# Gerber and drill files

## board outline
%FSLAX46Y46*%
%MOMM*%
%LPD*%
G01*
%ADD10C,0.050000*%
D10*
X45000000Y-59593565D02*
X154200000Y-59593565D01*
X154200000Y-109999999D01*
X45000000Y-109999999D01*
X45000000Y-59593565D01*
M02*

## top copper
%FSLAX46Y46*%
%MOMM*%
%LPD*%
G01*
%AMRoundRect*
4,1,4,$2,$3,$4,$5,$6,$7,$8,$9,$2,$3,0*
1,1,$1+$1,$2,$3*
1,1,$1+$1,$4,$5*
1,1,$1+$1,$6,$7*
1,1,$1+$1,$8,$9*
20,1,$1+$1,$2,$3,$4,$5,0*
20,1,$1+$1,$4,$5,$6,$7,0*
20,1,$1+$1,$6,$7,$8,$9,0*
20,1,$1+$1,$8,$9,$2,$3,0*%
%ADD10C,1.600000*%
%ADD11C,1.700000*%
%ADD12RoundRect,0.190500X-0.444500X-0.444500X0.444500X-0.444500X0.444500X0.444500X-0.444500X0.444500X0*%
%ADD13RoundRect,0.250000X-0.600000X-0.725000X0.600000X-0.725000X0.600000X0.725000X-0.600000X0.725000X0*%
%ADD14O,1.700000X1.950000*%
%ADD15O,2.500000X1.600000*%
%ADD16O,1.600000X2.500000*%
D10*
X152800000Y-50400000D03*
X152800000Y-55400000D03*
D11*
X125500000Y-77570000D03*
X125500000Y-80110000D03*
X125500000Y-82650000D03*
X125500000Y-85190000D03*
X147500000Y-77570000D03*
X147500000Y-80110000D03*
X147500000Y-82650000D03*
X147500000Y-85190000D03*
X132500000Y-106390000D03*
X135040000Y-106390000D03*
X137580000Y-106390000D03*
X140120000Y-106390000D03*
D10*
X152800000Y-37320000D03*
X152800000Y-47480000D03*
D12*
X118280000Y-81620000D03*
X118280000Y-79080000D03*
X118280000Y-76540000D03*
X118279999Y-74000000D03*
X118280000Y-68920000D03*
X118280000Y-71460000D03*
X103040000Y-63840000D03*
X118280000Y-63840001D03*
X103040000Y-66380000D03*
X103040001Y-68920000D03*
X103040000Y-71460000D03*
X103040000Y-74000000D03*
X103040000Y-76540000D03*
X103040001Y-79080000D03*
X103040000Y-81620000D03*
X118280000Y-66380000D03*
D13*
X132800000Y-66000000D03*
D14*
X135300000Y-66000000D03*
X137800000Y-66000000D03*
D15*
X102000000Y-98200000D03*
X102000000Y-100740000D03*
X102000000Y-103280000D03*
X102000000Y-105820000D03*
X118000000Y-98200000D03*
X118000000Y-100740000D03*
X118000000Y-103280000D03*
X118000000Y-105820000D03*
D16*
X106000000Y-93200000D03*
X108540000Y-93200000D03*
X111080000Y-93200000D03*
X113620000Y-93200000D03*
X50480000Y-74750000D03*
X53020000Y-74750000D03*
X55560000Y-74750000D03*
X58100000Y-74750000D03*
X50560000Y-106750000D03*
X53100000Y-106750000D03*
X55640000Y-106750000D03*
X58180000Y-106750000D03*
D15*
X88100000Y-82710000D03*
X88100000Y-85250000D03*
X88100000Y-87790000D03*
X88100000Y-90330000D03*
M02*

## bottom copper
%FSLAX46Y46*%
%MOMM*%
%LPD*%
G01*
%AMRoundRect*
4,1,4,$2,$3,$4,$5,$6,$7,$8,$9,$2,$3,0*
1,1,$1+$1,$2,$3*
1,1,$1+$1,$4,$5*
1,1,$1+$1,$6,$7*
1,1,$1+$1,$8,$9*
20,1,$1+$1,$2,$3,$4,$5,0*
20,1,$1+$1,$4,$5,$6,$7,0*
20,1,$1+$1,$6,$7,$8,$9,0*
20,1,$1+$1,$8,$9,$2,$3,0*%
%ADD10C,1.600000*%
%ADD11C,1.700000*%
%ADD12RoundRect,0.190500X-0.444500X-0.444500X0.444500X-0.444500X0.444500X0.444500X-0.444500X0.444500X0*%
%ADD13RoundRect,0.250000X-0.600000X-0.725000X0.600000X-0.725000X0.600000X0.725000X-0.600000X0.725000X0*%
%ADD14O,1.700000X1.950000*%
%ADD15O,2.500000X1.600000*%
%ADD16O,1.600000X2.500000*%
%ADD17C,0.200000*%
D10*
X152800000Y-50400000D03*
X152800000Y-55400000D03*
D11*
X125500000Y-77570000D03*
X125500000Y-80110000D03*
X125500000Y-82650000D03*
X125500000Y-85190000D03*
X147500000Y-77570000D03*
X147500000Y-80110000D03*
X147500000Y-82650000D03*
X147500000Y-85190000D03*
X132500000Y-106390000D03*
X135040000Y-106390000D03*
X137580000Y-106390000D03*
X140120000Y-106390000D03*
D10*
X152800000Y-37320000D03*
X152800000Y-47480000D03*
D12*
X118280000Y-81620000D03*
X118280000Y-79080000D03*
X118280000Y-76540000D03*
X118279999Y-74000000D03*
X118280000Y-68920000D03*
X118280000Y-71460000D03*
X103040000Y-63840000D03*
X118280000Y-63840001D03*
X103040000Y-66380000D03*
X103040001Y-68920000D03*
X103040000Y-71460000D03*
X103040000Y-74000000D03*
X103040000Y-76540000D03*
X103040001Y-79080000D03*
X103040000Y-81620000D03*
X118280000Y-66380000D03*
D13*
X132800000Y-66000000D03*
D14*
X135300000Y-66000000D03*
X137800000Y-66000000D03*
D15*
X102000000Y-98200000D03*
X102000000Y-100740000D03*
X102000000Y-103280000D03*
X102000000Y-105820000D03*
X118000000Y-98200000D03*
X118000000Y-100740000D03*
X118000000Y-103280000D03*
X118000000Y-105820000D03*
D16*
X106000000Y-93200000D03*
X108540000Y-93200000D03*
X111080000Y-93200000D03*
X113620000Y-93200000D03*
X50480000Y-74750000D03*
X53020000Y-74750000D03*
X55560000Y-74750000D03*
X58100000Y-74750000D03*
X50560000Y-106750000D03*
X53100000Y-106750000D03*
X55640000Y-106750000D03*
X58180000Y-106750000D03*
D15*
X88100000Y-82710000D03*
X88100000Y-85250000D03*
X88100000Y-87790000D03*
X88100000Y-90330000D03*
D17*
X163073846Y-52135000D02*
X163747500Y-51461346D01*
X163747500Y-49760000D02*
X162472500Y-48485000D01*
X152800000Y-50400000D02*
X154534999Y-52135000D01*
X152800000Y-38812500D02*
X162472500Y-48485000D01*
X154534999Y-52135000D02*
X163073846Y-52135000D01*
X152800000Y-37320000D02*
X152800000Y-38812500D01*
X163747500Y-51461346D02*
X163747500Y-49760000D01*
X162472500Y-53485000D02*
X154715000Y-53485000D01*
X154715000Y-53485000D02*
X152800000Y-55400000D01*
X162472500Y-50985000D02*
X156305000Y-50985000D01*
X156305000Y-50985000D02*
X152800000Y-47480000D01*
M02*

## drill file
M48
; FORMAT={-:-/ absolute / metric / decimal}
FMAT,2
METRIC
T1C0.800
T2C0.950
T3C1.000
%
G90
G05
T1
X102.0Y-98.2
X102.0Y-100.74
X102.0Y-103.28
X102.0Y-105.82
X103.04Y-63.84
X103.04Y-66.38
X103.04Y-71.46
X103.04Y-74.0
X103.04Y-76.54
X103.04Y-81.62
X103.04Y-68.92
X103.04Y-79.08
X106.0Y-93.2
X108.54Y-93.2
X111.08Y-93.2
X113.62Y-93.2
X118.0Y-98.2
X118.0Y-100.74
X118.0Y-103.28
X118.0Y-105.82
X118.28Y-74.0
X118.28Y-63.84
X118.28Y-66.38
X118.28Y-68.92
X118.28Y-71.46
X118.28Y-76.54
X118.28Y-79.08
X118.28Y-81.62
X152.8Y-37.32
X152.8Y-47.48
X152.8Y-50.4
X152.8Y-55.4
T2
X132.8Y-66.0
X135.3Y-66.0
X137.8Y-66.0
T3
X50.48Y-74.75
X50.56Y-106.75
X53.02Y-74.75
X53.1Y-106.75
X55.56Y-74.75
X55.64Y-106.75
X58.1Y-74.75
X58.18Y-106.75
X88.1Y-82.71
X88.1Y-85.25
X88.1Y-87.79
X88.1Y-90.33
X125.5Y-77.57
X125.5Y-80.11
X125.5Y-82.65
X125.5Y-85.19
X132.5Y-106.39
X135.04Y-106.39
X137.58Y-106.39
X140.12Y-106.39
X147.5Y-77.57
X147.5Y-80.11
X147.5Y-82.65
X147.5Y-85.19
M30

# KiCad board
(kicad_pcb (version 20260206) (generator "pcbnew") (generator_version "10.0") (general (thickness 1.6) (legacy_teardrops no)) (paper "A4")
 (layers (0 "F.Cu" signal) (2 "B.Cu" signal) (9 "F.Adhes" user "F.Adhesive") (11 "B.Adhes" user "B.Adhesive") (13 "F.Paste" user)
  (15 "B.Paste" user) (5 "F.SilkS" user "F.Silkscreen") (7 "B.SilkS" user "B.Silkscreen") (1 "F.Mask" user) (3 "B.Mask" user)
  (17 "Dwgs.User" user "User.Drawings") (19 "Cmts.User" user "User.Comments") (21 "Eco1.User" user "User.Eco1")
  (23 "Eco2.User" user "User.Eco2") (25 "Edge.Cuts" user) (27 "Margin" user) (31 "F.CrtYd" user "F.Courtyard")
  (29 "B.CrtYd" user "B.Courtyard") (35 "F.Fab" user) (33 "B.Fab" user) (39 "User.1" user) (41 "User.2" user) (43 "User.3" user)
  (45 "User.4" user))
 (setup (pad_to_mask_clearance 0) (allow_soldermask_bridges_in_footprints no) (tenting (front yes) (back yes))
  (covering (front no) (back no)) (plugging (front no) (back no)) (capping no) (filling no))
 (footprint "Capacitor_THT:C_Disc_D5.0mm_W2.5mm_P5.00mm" (layer "F.Cu") (at 152.8 50.4 -90)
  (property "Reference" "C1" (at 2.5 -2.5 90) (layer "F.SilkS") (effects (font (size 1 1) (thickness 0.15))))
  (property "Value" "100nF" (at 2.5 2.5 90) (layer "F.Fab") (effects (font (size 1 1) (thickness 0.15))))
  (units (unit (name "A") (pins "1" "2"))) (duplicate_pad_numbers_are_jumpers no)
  (pad "1" thru_hole circle (at 0 0 270) (size 1.6 1.6) (drill 0.8) (layers "*.Cu" "*.Mask") (remove_unused_layers no) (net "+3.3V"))
  (pad "2" thru_hole circle (at 5 0 270) (size 1.6 1.6) (drill 0.8) (layers "*.Cu" "*.Mask") (remove_unused_layers no) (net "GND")))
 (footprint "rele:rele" (layer "F.Cu") (at 137 89.15)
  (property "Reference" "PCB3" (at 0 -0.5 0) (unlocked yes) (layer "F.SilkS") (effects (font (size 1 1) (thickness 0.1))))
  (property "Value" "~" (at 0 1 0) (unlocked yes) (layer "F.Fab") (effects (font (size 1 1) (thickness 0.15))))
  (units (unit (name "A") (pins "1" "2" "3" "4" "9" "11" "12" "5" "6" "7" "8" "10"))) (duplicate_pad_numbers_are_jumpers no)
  (pad "1" thru_hole circle (at -11.5 -11.58 270) (size 1.7 1.7) (drill 1) (layers "*.Cu" "*.Mask") (remove_unused_layers no)
   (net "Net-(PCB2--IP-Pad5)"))
  (pad "2" thru_hole circle (at -11.5 -9.04 270) (size 1.7 1.7) (drill 1) (layers "*.Cu" "*.Mask") (remove_unused_layers no)
   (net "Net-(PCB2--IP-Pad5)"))
  (pad "3" thru_hole circle (at -11.5 -6.5 270) (size 1.7 1.7) (drill 1) (layers "*.Cu" "*.Mask") (remove_unused_layers no)
   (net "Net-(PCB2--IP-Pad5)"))
  (pad "4" thru_hole circle (at -11.5 -3.96 270) (size 1.7 1.7) (drill 1) (layers "*.Cu" "*.Mask") (remove_unused_layers no)
   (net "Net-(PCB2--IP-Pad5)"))
  (pad "5" thru_hole circle (at 10.5 -11.58 270) (size 1.7 1.7) (drill 1) (layers "*.Cu" "*.Mask") (remove_unused_layers no)
   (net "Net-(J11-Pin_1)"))
  (pad "6" thru_hole circle (at 10.5 -9.04 270) (size 1.7 1.7) (drill 1) (layers "*.Cu" "*.Mask") (remove_unused_layers no)
   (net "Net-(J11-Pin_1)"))
  (pad "7" thru_hole circle (at 10.5 -6.5 270) (size 1.7 1.7) (drill 1) (layers "*.Cu" "*.Mask") (remove_unused_layers no)
   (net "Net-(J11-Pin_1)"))
  (pad "8" thru_hole circle (at 10.5 -3.96 270) (size 1.7 1.7) (drill 1) (layers "*.Cu" "*.Mask") (remove_unused_layers no)
   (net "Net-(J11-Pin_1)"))
  (pad "9" thru_hole circle (at -4.5 17.24 180) (size 1.7 1.7) (drill 1) (layers "*.Cu" "*.Mask") (remove_unused_layers no) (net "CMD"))
  (pad "10" thru_hole circle (at -1.96 17.24 180) (size 1.7 1.7) (drill 1) (layers "*.Cu" "*.Mask") (remove_unused_layers no) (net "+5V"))
  (pad "11" thru_hole circle (at 0.58 17.24 180) (size 1.7 1.7) (drill 1) (layers "*.Cu" "*.Mask") (remove_unused_layers no) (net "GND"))
  (pad "12" thru_hole circle (at 3.12 17.24 180) (size 1.7 1.7) (drill 1) (layers "*.Cu" "*.Mask") (remove_unused_layers no) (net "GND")))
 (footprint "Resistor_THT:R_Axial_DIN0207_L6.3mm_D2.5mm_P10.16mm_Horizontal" (layer "F.Cu") (at 152.8 37.32 -90)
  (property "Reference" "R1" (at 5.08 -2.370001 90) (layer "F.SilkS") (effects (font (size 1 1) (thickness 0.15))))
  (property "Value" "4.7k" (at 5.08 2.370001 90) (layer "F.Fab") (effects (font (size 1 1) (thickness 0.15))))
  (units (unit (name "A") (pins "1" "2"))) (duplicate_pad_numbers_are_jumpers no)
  (pad "1" thru_hole circle (at 0 0 270) (size 1.6 1.6) (drill 0.8) (layers "*.Cu" "*.Mask") (remove_unused_layers no) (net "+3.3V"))
  (pad "2" thru_hole circle (at 10.16 0 270) (size 1.6 1.6) (drill 0.8) (layers "*.Cu" "*.Mask") (remove_unused_layers no)
   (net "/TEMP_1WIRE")))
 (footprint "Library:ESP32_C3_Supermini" (layer "F.Cu") (at 113.2 74)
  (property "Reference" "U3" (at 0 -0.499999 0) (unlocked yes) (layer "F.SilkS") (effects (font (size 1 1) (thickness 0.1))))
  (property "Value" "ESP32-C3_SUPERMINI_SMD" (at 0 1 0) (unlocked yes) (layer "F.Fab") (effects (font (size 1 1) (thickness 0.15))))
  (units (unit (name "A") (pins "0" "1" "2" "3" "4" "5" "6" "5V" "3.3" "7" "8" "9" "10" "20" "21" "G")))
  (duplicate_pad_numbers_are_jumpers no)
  (pad "0" thru_hole roundrect (at 5.08 7.62) (size 1.27 1.27) (drill 0.8) (layers "*.Cu" "*.Mask") (remove_unused_layers no)
   (roundrect_rratio 0.15) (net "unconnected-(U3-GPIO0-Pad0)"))
  (pad "1" thru_hole roundrect (at 5.08 5.08) (size 1.27 1.27) (drill 0.8) (layers "*.Cu" "*.Mask") (remove_unused_layers no)
   (roundrect_rratio 0.15) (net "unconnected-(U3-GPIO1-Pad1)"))
  (pad "2" thru_hole roundrect (at 5.08 2.54) (size 1.27 1.27) (drill 0.8) (layers "*.Cu" "*.Mask") (remove_unused_layers no)
   (roundrect_rratio 0.15) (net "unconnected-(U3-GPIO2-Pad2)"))
  (pad "3" thru_hole roundrect (at 5.079999 0) (size 1.27 1.27) (drill 0.8) (layers "*.Cu" "*.Mask") (remove_unused_layers no)
   (roundrect_rratio 0.15) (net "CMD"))
  (pad "3.3" thru_hole roundrect (at 5.08 -5.08) (size 1.27 1.27) (drill 0.8) (layers "*.Cu" "*.Mask") (remove_unused_layers no)
   (roundrect_rratio 0.15) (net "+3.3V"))
  (pad "4" thru_hole roundrect (at 5.08 -2.54) (size 1.27 1.27) (drill 0.8) (layers "*.Cu" "*.Mask") (remove_unused_layers no)
   (roundrect_rratio 0.15) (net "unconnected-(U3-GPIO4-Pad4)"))
  (pad "5" thru_hole roundrect (at -10.16 -10.16) (size 1.27 1.27) (drill 0.8) (layers "*.Cu" "*.Mask") (remove_unused_layers no)
   (roundrect_rratio 0.15) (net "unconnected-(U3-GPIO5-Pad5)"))
  (pad "5V" thru_hole roundrect (at 5.08 -10.159999) (size 1.27 1.27) (drill 0.8) (layers "*.Cu" "*.Mask") (remove_unused_layers no)
   (roundrect_rratio 0.15) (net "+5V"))
  (pad "6" thru_hole roundrect (at -10.16 -7.62) (size 1.27 1.27) (drill 0.8) (layers "*.Cu" "*.Mask") (remove_unused_layers no)
   (roundrect_rratio 0.15) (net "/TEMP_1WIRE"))
  (pad "7" thru_hole roundrect (at -10.159999 -5.08) (size 1.27 1.27) (drill 0.8) (layers "*.Cu" "*.Mask") (remove_unused_layers no)
   (roundrect_rratio 0.15) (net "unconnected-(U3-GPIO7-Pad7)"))
  (pad "8" thru_hole roundrect (at -10.16 -2.54) (size 1.27 1.27) (drill 0.8) (layers "*.Cu" "*.Mask") (remove_unused_layers no)
   (roundrect_rratio 0.15) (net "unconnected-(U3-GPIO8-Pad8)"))
  (pad "9" thru_hole roundrect (at -10.16 0) (size 1.27 1.27) (drill 0.8) (layers "*.Cu" "*.Mask") (remove_unused_layers no)
   (roundrect_rratio 0.15) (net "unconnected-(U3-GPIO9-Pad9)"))
  (pad "10" thru_hole roundrect (at -10.16 2.54) (size 1.27 1.27) (drill 0.8) (layers "*.Cu" "*.Mask") (remove_unused_layers no)
   (roundrect_rratio 0.15) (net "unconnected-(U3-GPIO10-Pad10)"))
  (pad "20" thru_hole roundrect (at -10.159999 5.08) (size 1.27 1.27) (drill 0.8) (layers "*.Cu" "*.Mask") (remove_unused_layers no)
   (roundrect_rratio 0.15) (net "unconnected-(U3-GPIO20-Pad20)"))
  (pad "21" thru_hole roundrect (at -10.16 7.62) (size 1.27 1.27) (drill 0.8) (layers "*.Cu" "*.Mask") (remove_unused_layers no)
   (roundrect_rratio 0.15) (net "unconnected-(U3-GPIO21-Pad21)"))
  (pad "G" thru_hole roundrect (at 5.08 -7.62) (size 1.27 1.27) (drill 0.8) (layers "*.Cu" "*.Mask") (remove_unused_layers no)
   (roundrect_rratio 0.15) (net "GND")))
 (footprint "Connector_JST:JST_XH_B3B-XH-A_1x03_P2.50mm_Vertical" (layer "F.Cu") (at 132.8 66)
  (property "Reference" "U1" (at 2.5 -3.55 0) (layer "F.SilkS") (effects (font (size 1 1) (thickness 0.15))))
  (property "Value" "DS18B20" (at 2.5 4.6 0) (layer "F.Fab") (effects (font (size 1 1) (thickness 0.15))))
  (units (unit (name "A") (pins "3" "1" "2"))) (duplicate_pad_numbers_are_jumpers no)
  (pad "1" thru_hole roundrect (at 0 0) (size 1.7 1.95) (drill 0.95) (layers "*.Cu" "*.Mask") (remove_unused_layers no)
   (roundrect_rratio 0.147059) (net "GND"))
  (pad "2" thru_hole oval (at 2.5 0) (size 1.7 1.95) (drill 0.95) (layers "*.Cu" "*.Mask") (remove_unused_layers no) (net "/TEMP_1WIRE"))
  (pad "3" thru_hole oval (at 5 0) (size 1.7 1.95) (drill 0.95) (layers "*.Cu" "*.Mask") (remove_unused_layers no) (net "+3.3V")))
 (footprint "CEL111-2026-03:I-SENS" (layer "F.Cu") (at 110 90.7)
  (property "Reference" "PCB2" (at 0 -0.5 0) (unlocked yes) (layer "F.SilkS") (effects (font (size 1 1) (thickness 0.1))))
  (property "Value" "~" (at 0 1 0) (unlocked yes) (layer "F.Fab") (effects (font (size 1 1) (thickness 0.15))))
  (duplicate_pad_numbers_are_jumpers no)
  (pad "1" thru_hole oval (at -8 7.5 270) (size 1.6 2.5) (drill 0.8) (layers "*.Cu" "*.Mask") (remove_unused_layers no) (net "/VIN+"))
  (pad "2" thru_hole oval (at -8 10.04 270) (size 1.6 2.5) (drill 0.8) (layers "*.Cu" "*.Mask") (remove_unused_layers no) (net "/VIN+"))
  (pad "3" thru_hole oval (at -8 12.58 270) (size 1.6 2.5) (drill 0.8) (layers "*.Cu" "*.Mask") (remove_unused_layers no) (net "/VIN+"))
  (pad "4" thru_hole oval (at -8 15.12 270) (size 1.6 2.5) (drill 0.8) (layers "*.Cu" "*.Mask") (remove_unused_layers no) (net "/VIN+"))
  (pad "5" thru_hole oval (at 8 7.5 270) (size 1.6 2.5) (drill 0.8) (layers "*.Cu" "*.Mask") (remove_unused_layers no)
   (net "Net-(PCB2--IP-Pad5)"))
  (pad "6" thru_hole oval (at 8 10.04 270) (size 1.6 2.5) (drill 0.8) (layers "*.Cu" "*.Mask") (remove_unused_layers no)
   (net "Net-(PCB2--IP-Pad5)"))
  (pad "7" thru_hole oval (at 8 12.58 270) (size 1.6 2.5) (drill 0.8) (layers "*.Cu" "*.Mask") (remove_unused_layers no)
   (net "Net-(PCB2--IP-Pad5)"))
  (pad "8" thru_hole oval (at 8 15.12 270) (size 1.6 2.5) (drill 0.8) (layers "*.Cu" "*.Mask") (remove_unused_layers no)
   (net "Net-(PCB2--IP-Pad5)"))
  (pad "9" thru_hole oval (at -4 2.5) (size 1.6 2.5) (drill 0.8) (layers "*.Cu" "*.Mask") (remove_unused_layers no) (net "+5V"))
  (pad "10" thru_hole oval (at -1.46 2.5) (size 1.6 2.5) (drill 0.8) (layers "*.Cu" "*.Mask") (remove_unused_layers no) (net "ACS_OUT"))
  (pad "11" thru_hole oval (at 1.08 2.5) (size 1.6 2.5) (drill 0.8) (layers "*.Cu" "*.Mask") (remove_unused_layers no) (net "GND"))
  (pad "12" thru_hole oval (at 3.62 2.5) (size 1.6 2.5) (drill 0.8) (layers "*.Cu" "*.Mask") (remove_unused_layers no) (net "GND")))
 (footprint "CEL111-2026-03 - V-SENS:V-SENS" (layer "F.Cu") (at 72.6 72.25)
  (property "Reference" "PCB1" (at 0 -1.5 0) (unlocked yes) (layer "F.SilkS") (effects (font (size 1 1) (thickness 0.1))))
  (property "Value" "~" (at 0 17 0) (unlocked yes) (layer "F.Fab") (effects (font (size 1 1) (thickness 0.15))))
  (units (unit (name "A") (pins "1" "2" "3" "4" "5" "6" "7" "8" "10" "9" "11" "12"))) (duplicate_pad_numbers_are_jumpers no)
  (pad "1" thru_hole oval (at -22.12 2.5) (size 1.6 2.5) (drill 1) (layers "*.Cu" "*.Mask") (remove_unused_layers no) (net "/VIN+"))
  (pad "2" thru_hole oval (at -19.58 2.5) (size 1.6 2.5) (drill 1) (layers "*.Cu" "*.Mask") (remove_unused_layers no) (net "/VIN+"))
  (pad "3" thru_hole oval (at -17.04 2.5) (size 1.6 2.5) (drill 1) (layers "*.Cu" "*.Mask") (remove_unused_layers no) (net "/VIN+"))
  (pad "4" thru_hole oval (at -14.5 2.5) (size 1.6 2.5) (drill 1) (layers "*.Cu" "*.Mask") (remove_unused_layers no) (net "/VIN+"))
  (pad "5" thru_hole oval (at -22.04 34.5) (size 1.6 2.5) (drill 1) (layers "*.Cu" "*.Mask") (remove_unused_layers no) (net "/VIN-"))
  (pad "6" thru_hole oval (at -19.5 34.5) (size 1.6 2.5) (drill 1) (layers "*.Cu" "*.Mask") (remove_unused_layers no) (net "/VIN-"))
  (pad "7" thru_hole oval (at -16.96 34.5) (size 1.6 2.5) (drill 1) (layers "*.Cu" "*.Mask") (remove_unused_layers no) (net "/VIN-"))
  (pad "8" thru_hole oval (at -14.42 34.5) (size 1.6 2.5) (drill 1) (layers "*.Cu" "*.Mask") (remove_unused_layers no) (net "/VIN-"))
  (pad "9" thru_hole oval (at 15.5 10.46 270) (size 1.6 2.5) (drill 1) (layers "*.Cu" "*.Mask") (remove_unused_layers no) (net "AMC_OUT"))
  (pad "10" thru_hole oval (at 15.5 13 270) (size 1.6 2.5) (drill 1) (layers "*.Cu" "*.Mask") (remove_unused_layers no) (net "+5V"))
  (pad "11" thru_hole oval (at 15.5 15.54 270) (size 1.6 2.5) (drill 1) (layers "*.Cu" "*.Mask") (remove_unused_layers no) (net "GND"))
  (pad "12" thru_hole oval (at 15.5 18.08 270) (size 1.6 2.5) (drill 1) (layers "*.Cu" "*.Mask") (remove_unused_layers no) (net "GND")))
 (gr_rect (start 45 59.593565) (end 154.2 109.999999) (stroke (width 0.05) (type solid)) (fill no) (layer "Edge.Cuts"))
 (segment (start 163.073846 52.135) (end 163.7475 51.461346) (width 0.2) (layer "B.Cu") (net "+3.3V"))
 (segment (start 163.7475 49.76) (end 162.4725 48.485) (width 0.2) (layer "B.Cu") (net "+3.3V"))
 (segment (start 152.8 50.4) (end 154.534999 52.135) (width 0.2) (layer "B.Cu") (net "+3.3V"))
 (segment (start 152.8 38.8125) (end 162.4725 48.485) (width 0.2) (layer "B.Cu") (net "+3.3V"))
 (segment (start 154.534999 52.135) (end 163.073846 52.135) (width 0.2) (layer "B.Cu") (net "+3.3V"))
 (segment (start 152.8 37.32) (end 152.8 38.8125) (width 0.2) (layer "B.Cu") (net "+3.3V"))
 (segment (start 163.7475 51.461346) (end 163.7475 49.76) (width 0.2) (layer "B.Cu") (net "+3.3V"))
 (segment (start 162.4725 53.485) (end 154.715 53.485) (width 0.2) (layer "B.Cu") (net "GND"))
 (segment (start 154.715 53.485) (end 152.8 55.4) (width 0.2) (layer "B.Cu") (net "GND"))
 (segment (start 162.4725 50.985) (end 156.305 50.985) (width 0.2) (layer "B.Cu") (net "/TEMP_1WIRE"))
 (segment (start 156.305 50.985) (end 152.8 47.48) (width 0.2) (layer "B.Cu") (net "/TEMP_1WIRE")))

